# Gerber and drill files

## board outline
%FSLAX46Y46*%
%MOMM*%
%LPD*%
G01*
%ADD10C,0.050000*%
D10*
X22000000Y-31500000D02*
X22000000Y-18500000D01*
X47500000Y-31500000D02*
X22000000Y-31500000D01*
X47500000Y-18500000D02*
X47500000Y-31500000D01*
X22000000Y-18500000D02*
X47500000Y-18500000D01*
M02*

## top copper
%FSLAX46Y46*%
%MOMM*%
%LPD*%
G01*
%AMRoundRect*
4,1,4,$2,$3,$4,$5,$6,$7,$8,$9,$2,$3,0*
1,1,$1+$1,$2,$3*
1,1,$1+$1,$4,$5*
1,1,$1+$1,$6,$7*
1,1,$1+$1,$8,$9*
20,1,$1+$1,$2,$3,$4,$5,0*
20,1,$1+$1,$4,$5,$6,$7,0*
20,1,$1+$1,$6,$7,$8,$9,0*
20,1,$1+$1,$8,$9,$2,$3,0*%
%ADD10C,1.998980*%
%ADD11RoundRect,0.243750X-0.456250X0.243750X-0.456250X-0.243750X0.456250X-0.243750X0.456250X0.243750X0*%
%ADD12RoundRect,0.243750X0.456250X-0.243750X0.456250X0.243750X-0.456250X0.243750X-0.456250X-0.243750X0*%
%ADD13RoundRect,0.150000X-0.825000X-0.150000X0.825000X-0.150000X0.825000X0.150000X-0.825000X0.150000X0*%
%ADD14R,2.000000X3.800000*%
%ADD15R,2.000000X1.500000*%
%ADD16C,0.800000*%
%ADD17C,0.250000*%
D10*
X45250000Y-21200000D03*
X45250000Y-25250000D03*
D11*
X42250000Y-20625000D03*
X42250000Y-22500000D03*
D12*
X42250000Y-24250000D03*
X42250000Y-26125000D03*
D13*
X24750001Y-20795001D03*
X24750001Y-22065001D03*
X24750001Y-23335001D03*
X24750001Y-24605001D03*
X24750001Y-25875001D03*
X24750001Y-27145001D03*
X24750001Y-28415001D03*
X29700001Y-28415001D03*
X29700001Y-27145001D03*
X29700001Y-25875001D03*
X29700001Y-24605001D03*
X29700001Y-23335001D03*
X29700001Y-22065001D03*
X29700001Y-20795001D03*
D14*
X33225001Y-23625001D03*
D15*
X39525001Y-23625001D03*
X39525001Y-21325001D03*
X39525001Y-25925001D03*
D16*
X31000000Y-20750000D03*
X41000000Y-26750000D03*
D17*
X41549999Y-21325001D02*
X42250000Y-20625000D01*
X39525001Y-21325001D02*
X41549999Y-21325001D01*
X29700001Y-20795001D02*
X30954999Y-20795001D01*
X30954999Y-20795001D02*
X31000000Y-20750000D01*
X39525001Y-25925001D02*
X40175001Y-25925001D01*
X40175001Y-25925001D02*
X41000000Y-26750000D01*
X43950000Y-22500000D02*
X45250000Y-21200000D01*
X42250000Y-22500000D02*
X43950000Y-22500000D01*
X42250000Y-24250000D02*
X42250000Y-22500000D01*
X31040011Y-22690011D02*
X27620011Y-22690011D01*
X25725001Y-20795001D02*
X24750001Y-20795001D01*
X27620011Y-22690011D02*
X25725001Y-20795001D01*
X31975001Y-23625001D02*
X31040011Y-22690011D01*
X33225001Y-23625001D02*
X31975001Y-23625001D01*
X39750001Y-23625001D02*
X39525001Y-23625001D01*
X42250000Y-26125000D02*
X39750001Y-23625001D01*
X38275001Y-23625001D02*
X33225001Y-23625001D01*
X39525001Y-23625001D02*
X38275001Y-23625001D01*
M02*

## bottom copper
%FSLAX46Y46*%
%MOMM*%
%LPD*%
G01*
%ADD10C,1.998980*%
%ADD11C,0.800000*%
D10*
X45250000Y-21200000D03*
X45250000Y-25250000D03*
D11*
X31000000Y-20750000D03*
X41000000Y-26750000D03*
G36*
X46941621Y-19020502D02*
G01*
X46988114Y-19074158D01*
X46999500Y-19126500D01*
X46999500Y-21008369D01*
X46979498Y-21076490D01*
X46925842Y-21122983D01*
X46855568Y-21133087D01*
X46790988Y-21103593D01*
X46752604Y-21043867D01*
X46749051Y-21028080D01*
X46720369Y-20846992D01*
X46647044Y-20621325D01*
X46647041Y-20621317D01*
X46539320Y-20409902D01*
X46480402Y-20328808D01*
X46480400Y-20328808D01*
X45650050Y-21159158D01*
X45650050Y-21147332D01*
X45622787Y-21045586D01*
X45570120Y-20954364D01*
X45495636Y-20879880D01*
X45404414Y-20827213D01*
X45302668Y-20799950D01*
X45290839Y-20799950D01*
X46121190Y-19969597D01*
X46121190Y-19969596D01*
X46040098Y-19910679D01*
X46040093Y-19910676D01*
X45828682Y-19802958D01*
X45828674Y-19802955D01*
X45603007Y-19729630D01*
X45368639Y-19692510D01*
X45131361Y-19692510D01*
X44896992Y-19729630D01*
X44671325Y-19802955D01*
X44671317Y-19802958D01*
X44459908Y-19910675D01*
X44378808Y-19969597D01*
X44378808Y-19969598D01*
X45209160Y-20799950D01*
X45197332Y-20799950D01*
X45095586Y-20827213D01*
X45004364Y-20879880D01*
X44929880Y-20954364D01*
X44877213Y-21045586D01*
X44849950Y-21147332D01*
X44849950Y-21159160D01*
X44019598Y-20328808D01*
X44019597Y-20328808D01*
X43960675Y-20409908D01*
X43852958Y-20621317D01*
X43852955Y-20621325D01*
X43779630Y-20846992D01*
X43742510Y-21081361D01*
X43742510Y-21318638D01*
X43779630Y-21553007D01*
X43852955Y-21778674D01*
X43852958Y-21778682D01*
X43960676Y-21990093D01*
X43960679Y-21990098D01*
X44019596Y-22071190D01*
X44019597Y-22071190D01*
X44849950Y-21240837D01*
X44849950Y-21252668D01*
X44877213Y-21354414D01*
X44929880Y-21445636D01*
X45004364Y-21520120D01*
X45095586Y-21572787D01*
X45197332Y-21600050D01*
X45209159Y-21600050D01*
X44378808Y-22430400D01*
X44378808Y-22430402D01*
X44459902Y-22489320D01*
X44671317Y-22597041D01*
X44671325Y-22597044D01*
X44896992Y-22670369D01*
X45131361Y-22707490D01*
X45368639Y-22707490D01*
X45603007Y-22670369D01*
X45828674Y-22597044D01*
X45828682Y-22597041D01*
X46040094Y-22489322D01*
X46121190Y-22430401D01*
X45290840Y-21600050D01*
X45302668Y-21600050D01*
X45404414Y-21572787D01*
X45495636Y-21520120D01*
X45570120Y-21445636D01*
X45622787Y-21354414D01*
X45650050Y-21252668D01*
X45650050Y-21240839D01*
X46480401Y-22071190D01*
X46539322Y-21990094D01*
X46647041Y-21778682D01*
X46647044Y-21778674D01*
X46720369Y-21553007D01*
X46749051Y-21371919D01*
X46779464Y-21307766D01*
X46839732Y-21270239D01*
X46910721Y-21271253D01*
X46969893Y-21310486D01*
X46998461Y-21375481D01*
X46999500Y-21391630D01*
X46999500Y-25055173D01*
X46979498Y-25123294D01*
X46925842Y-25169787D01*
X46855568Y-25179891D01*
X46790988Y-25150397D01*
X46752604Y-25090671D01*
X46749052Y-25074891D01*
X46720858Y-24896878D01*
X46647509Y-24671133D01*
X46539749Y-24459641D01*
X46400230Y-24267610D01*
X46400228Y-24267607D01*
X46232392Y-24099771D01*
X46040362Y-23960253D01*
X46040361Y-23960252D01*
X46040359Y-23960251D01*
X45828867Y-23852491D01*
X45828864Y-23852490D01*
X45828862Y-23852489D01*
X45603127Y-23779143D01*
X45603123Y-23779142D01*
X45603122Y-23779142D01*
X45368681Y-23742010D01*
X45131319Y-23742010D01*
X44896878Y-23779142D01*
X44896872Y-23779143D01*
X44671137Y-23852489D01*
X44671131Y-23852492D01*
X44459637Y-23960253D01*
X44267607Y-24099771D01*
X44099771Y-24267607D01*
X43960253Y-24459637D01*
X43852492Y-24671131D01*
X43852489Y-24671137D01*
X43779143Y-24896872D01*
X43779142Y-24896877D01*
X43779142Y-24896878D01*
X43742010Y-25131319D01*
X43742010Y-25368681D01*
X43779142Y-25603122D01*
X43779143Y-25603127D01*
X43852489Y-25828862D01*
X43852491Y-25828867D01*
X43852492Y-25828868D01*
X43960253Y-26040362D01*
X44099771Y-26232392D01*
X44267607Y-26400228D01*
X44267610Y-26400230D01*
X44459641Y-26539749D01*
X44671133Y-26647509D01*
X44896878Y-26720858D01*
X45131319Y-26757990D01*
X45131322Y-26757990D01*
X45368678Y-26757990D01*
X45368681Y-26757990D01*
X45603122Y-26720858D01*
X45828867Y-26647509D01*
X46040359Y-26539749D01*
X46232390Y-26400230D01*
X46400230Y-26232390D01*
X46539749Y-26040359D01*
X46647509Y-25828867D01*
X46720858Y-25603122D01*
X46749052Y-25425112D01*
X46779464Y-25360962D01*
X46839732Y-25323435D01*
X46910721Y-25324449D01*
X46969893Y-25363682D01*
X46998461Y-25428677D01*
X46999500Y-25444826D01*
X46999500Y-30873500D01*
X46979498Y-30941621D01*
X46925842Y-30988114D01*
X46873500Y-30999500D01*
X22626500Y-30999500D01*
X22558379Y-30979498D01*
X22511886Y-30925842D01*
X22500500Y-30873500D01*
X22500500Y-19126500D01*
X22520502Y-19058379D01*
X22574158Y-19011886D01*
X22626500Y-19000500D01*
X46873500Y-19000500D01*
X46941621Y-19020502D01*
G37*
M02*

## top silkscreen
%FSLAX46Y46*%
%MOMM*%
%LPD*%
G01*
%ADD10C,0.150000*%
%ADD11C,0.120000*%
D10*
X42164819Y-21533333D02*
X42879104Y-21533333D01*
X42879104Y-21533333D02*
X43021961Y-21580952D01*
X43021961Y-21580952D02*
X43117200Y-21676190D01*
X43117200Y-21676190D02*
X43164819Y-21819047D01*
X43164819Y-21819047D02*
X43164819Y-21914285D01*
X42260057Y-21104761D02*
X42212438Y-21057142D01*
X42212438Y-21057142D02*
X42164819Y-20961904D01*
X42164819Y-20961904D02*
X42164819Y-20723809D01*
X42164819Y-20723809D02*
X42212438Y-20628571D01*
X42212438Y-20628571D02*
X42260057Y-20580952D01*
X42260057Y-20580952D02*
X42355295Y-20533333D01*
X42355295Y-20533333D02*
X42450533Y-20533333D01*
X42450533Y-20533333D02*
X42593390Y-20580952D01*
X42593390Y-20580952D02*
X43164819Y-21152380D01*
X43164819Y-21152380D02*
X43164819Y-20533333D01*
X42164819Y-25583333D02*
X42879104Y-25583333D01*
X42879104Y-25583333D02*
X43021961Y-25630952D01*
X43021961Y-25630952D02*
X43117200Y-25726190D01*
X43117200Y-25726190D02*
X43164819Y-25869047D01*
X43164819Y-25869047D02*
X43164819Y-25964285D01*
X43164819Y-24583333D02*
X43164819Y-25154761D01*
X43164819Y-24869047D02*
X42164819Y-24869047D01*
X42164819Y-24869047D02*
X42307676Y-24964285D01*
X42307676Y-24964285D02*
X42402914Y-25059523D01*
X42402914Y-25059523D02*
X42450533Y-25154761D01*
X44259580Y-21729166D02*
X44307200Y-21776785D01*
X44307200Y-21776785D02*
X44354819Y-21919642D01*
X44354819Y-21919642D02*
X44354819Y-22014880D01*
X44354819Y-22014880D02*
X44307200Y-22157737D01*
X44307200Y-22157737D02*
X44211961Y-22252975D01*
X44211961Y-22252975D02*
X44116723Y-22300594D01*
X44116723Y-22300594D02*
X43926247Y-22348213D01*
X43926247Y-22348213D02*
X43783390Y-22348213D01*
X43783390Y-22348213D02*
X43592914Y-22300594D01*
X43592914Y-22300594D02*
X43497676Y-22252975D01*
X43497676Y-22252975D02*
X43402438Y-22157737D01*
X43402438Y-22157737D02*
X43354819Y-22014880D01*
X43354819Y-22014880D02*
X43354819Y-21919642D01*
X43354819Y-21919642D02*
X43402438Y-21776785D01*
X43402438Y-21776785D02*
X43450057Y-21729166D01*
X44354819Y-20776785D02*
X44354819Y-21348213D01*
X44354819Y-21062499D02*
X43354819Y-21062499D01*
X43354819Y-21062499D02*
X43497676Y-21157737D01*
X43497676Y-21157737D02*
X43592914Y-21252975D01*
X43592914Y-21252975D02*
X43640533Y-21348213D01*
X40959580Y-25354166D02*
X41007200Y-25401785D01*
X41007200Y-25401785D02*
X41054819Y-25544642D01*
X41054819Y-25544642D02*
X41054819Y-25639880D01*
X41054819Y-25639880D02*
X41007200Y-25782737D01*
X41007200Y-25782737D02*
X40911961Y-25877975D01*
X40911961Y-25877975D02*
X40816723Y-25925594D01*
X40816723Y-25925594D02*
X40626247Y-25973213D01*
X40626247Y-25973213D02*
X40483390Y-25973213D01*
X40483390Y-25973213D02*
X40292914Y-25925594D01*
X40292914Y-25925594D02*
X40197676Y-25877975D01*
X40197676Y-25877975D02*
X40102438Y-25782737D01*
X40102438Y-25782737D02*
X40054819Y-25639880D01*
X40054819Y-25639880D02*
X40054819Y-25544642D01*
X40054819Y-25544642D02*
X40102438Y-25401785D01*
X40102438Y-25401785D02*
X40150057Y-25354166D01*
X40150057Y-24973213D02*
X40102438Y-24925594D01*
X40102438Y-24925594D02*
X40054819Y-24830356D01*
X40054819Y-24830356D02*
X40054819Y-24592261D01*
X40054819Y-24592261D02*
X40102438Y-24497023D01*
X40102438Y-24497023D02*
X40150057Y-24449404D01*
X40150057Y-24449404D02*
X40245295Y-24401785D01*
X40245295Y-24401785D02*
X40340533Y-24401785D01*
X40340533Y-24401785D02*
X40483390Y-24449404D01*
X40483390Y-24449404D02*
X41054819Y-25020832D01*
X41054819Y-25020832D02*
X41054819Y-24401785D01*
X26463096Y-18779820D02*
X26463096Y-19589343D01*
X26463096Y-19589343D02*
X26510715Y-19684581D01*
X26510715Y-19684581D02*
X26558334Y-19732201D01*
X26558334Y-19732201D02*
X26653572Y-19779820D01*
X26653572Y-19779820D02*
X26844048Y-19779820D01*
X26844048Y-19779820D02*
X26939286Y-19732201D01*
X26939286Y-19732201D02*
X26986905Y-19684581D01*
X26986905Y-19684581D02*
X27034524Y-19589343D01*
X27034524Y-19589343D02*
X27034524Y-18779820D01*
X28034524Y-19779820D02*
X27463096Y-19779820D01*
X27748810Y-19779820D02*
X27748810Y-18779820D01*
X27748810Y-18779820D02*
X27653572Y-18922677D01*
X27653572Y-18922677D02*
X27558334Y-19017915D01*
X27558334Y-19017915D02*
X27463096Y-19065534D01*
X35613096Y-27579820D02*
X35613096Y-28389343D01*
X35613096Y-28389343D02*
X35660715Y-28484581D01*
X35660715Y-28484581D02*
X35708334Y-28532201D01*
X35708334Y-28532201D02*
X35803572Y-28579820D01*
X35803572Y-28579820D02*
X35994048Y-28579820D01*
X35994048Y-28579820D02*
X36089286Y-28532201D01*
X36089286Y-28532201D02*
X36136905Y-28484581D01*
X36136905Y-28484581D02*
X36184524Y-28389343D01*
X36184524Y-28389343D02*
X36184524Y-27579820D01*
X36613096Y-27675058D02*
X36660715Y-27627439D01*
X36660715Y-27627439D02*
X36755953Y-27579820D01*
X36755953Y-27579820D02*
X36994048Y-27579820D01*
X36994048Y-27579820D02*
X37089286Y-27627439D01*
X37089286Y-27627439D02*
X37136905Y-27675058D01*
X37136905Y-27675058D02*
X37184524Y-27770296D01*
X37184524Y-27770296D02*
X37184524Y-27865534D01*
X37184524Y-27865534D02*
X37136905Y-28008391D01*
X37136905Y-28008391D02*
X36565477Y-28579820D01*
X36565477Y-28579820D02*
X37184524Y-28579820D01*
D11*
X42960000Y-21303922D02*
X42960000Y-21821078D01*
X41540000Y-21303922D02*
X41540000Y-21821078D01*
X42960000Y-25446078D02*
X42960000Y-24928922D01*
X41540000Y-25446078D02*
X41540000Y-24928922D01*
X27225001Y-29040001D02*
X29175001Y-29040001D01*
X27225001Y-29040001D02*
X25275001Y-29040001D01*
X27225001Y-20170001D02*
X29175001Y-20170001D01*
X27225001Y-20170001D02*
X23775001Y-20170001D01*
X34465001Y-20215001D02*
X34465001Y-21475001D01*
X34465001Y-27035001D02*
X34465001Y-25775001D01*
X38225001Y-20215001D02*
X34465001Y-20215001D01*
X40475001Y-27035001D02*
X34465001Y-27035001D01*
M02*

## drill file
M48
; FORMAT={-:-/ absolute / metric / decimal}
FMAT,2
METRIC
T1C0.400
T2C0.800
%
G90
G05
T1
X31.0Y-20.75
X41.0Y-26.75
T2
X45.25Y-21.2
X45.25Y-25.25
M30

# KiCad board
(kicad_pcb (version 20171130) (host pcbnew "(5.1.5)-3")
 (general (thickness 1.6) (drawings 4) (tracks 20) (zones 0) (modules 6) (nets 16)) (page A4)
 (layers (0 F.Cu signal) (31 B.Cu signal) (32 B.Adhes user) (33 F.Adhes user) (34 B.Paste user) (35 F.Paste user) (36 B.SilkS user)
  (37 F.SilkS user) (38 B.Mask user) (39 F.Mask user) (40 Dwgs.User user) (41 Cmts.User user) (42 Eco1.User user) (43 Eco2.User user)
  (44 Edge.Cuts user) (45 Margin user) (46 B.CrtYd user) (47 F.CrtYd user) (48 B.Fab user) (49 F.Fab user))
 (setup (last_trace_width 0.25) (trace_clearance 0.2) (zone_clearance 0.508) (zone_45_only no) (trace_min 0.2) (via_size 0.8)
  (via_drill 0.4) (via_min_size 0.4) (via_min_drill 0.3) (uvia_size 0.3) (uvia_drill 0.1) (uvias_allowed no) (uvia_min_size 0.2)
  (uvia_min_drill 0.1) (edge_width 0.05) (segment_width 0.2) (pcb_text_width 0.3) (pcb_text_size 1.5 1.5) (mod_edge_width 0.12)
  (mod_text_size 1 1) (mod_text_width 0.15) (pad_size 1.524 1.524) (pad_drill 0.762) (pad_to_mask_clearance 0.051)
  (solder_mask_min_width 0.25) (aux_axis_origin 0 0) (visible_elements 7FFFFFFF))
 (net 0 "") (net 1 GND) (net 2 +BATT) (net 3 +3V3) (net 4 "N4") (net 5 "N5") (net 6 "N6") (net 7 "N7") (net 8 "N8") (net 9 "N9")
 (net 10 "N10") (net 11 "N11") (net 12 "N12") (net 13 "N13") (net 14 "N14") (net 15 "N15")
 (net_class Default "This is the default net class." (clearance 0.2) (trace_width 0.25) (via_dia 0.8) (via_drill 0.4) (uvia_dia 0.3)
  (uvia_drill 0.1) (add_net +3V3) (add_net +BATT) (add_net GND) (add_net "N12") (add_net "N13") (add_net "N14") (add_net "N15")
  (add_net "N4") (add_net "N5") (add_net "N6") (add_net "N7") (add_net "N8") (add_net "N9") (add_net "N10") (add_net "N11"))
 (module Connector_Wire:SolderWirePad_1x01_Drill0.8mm (layer F.Cu) (at 45.25 21.2 90)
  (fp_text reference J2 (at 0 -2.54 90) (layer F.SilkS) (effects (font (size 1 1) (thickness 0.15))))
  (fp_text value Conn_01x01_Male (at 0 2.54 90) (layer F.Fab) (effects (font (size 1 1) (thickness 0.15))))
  (pad 1 thru_hole circle (at 0 0 90) (size 1.99898 1.99898) (drill 0.8001) (layers *.Cu *.Mask) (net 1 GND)))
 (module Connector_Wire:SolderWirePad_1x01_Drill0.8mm (layer F.Cu) (at 45.25 25.25 90)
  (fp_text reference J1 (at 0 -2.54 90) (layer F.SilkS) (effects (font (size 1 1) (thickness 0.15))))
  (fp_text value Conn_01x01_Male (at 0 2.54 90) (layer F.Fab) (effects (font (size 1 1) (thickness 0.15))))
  (pad 1 thru_hole circle (at 0 0 90) (size 1.99898 1.99898) (drill 0.8001) (layers *.Cu *.Mask) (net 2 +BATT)))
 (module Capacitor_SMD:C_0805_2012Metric (layer F.Cu) (at 42.25 21.5625 270)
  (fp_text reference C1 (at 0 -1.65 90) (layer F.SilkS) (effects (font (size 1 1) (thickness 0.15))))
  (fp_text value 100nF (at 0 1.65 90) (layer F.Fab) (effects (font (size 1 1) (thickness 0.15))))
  (fp_line (start -0.258578 -0.71) (end 0.258578 -0.71) (layer F.SilkS) (width 0.12))
  (fp_line (start -0.258578 0.71) (end 0.258578 0.71) (layer F.SilkS) (width 0.12))
  (pad 1 smd roundrect (at -0.9375 0 270) (size 0.975 1.4) (layers F.Cu F.Paste F.Mask) (roundrect_rratio 0.25) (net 2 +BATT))
  (pad 2 smd roundrect (at 0.9375 0 270) (size 0.975 1.4) (layers F.Cu F.Paste F.Mask) (roundrect_rratio 0.25) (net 1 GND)))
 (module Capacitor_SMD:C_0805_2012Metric (layer F.Cu) (at 42.25 25.1875 90)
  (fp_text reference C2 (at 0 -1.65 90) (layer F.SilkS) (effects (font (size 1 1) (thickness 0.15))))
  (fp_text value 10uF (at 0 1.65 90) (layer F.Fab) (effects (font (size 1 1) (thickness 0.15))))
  (fp_line (start -0.258578 0.71) (end 0.258578 0.71) (layer F.SilkS) (width 0.12))
  (fp_line (start -0.258578 -0.71) (end 0.258578 -0.71) (layer F.SilkS) (width 0.12))
  (pad 2 smd roundrect (at 0.9375 0 90) (size 0.975 1.4) (layers F.Cu F.Paste F.Mask) (roundrect_rratio 0.25) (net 1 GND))
  (pad 1 smd roundrect (at -0.9375 0 90) (size 0.975 1.4) (layers F.Cu F.Paste F.Mask) (roundrect_rratio 0.25) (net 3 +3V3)))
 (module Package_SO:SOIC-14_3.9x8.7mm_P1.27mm (layer F.Cu) (at 27.225001 24.605001)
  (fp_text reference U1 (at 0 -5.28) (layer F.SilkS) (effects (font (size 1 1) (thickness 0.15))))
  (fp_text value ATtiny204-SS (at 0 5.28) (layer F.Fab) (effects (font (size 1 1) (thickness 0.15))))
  (fp_line (start 0 4.435) (end 1.95 4.435) (layer F.SilkS) (width 0.12))
  (fp_line (start 0 4.435) (end -1.95 4.435) (layer F.SilkS) (width 0.12))
  (fp_line (start 0 -4.435) (end 1.95 -4.435) (layer F.SilkS) (width 0.12))
  (fp_line (start 0 -4.435) (end -3.45 -4.435) (layer F.SilkS) (width 0.12))
  (pad 1 smd roundrect (at -2.475 -3.81) (size 1.95 0.6) (layers F.Cu F.Paste F.Mask) (roundrect_rratio 0.25) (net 3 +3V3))
  (pad 2 smd roundrect (at -2.475 -2.54) (size 1.95 0.6) (layers F.Cu F.Paste F.Mask) (roundrect_rratio 0.25) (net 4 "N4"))
  (pad 3 smd roundrect (at -2.475 -1.27) (size 1.95 0.6) (layers F.Cu F.Paste F.Mask) (roundrect_rratio 0.25) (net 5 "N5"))
  (pad 4 smd roundrect (at -2.475 0) (size 1.95 0.6) (layers F.Cu F.Paste F.Mask) (roundrect_rratio 0.25) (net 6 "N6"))
  (pad 5 smd roundrect (at -2.475 1.27) (size 1.95 0.6) (layers F.Cu F.Paste F.Mask) (roundrect_rratio 0.25) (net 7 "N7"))
  (pad 6 smd roundrect (at -2.475 2.54) (size 1.95 0.6) (layers F.Cu F.Paste F.Mask) (roundrect_rratio 0.25) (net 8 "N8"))
  (pad 7 smd roundrect (at -2.475 3.81) (size 1.95 0.6) (layers F.Cu F.Paste F.Mask) (roundrect_rratio 0.25) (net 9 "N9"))
  (pad 8 smd roundrect (at 2.475 3.81) (size 1.95 0.6) (layers F.Cu F.Paste F.Mask) (roundrect_rratio 0.25) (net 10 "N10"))
  (pad 9 smd roundrect (at 2.475 2.54) (size 1.95 0.6) (layers F.Cu F.Paste F.Mask) (roundrect_rratio 0.25) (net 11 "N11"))
  (pad 10 smd roundrect (at 2.475 1.27) (size 1.95 0.6) (layers F.Cu F.Paste F.Mask) (roundrect_rratio 0.25) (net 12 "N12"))
  (pad 11 smd roundrect (at 2.475 0) (size 1.95 0.6) (layers F.Cu F.Paste F.Mask) (roundrect_rratio 0.25) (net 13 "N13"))
  (pad 12 smd roundrect (at 2.475 -1.27) (size 1.95 0.6) (layers F.Cu F.Paste F.Mask) (roundrect_rratio 0.25) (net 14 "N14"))
  (pad 13 smd roundrect (at 2.475 -2.54) (size 1.95 0.6) (layers F.Cu F.Paste F.Mask) (roundrect_rratio 0.25) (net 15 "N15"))
  (pad 14 smd roundrect (at 2.475 -3.81) (size 1.95 0.6) (layers F.Cu F.Paste F.Mask) (roundrect_rratio 0.25) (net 1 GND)))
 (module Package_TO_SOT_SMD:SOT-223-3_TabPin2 (layer F.Cu) (at 36.375001 23.625001 180)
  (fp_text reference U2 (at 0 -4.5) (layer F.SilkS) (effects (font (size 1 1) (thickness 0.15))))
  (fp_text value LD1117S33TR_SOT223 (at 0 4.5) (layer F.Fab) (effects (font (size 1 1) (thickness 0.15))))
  (fp_line (start 1.91 3.41) (end 1.91 2.15) (layer F.SilkS) (width 0.12))
  (fp_line (start 1.91 -3.41) (end 1.91 -2.15) (layer F.SilkS) (width 0.12))
  (fp_line (start -1.85 3.41) (end 1.91 3.41) (layer F.SilkS) (width 0.12))
  (fp_line (start -4.1 -3.41) (end 1.91 -3.41) (layer F.SilkS) (width 0.12))
  (pad 2 smd rect (at 3.15 0 180) (size 2 3.8) (layers F.Cu F.Paste F.Mask) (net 3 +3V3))
  (pad 2 smd rect (at -3.15 0 180) (size 2 1.5) (layers F.Cu F.Paste F.Mask) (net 3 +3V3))
  (pad 3 smd rect (at -3.15 2.3 180) (size 2 1.5) (layers F.Cu F.Paste F.Mask) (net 2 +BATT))
  (pad 1 smd rect (at -3.15 -2.3 180) (size 2 1.5) (layers F.Cu F.Paste F.Mask) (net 1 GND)))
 (gr_line (start 22 31.5) (end 22 18.5) (layer Edge.Cuts) (width 0.05))
 (gr_line (start 47.5 31.5) (end 22 31.5) (layer Edge.Cuts) (width 0.05))
 (gr_line (start 47.5 18.5) (end 47.5 31.5) (layer Edge.Cuts) (width 0.05))
 (gr_line (start 22 18.5) (end 47.5 18.5) (layer Edge.Cuts) (width 0.05))
 (segment (start 41.549999 21.325001) (end 42.25 20.625) (width 0.25) (layer F.Cu) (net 2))
 (segment (start 39.525001 21.325001) (end 41.549999 21.325001) (width 0.25) (layer F.Cu) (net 2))
 (segment (start 29.700001 20.795001) (end 30.954999 20.795001) (width 0.25) (layer F.Cu) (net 1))
 (via (at 31 20.75) (size 0.8) (drill 0.4) (layers F.Cu B.Cu) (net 1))
 (segment (start 30.954999 20.795001) (end 31 20.75) (width 0.25) (layer F.Cu) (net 1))
 (via (at 41 26.75) (size 0.8) (drill 0.4) (layers F.Cu B.Cu) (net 1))
 (segment (start 39.525001 25.925001) (end 40.175001 25.925001) (width 0.25) (layer F.Cu) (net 1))
 (segment (start 40.175001 25.925001) (end 41 26.75) (width 0.25) (layer F.Cu) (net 1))
 (segment (start 43.95 22.5) (end 45.25 21.2) (width 0.25) (layer F.Cu) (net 1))
 (segment (start 42.25 22.5) (end 43.95 22.5) (width 0.25) (layer F.Cu) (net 1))
 (segment (start 42.25 24.25) (end 42.25 22.5) (width 0.25) (layer F.Cu) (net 1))
 (segment (start 31.040011 22.690011) (end 27.620011 22.690011) (width 0.25) (layer F.Cu) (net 3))
 (segment (start 25.725001 20.795001) (end 24.750001 20.795001) (width 0.25) (layer F.Cu) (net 3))
 (segment (start 27.620011 22.690011) (end 25.725001 20.795001) (width 0.25) (layer F.Cu) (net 3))
 (segment (start 31.975001 23.625001) (end 31.040011 22.690011) (width 0.25) (layer F.Cu) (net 3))
 (segment (start 33.225001 23.625001) (end 31.975001 23.625001) (width 0.25) (layer F.Cu) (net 3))
 (segment (start 39.750001 23.625001) (end 39.525001 23.625001) (width 0.25) (layer F.Cu) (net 3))
 (segment (start 42.25 26.125) (end 39.750001 23.625001) (width 0.25) (layer F.Cu) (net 3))
 (segment (start 38.275001 23.625001) (end 33.225001 23.625001) (width 0.25) (layer F.Cu) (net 3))
 (segment (start 39.525001 23.625001) (end 38.275001 23.625001) (width 0.25) (layer F.Cu) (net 3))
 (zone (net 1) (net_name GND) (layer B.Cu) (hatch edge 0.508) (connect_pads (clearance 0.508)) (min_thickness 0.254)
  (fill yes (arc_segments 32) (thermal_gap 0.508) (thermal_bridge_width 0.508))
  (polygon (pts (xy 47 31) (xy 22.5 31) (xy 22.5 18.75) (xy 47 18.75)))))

